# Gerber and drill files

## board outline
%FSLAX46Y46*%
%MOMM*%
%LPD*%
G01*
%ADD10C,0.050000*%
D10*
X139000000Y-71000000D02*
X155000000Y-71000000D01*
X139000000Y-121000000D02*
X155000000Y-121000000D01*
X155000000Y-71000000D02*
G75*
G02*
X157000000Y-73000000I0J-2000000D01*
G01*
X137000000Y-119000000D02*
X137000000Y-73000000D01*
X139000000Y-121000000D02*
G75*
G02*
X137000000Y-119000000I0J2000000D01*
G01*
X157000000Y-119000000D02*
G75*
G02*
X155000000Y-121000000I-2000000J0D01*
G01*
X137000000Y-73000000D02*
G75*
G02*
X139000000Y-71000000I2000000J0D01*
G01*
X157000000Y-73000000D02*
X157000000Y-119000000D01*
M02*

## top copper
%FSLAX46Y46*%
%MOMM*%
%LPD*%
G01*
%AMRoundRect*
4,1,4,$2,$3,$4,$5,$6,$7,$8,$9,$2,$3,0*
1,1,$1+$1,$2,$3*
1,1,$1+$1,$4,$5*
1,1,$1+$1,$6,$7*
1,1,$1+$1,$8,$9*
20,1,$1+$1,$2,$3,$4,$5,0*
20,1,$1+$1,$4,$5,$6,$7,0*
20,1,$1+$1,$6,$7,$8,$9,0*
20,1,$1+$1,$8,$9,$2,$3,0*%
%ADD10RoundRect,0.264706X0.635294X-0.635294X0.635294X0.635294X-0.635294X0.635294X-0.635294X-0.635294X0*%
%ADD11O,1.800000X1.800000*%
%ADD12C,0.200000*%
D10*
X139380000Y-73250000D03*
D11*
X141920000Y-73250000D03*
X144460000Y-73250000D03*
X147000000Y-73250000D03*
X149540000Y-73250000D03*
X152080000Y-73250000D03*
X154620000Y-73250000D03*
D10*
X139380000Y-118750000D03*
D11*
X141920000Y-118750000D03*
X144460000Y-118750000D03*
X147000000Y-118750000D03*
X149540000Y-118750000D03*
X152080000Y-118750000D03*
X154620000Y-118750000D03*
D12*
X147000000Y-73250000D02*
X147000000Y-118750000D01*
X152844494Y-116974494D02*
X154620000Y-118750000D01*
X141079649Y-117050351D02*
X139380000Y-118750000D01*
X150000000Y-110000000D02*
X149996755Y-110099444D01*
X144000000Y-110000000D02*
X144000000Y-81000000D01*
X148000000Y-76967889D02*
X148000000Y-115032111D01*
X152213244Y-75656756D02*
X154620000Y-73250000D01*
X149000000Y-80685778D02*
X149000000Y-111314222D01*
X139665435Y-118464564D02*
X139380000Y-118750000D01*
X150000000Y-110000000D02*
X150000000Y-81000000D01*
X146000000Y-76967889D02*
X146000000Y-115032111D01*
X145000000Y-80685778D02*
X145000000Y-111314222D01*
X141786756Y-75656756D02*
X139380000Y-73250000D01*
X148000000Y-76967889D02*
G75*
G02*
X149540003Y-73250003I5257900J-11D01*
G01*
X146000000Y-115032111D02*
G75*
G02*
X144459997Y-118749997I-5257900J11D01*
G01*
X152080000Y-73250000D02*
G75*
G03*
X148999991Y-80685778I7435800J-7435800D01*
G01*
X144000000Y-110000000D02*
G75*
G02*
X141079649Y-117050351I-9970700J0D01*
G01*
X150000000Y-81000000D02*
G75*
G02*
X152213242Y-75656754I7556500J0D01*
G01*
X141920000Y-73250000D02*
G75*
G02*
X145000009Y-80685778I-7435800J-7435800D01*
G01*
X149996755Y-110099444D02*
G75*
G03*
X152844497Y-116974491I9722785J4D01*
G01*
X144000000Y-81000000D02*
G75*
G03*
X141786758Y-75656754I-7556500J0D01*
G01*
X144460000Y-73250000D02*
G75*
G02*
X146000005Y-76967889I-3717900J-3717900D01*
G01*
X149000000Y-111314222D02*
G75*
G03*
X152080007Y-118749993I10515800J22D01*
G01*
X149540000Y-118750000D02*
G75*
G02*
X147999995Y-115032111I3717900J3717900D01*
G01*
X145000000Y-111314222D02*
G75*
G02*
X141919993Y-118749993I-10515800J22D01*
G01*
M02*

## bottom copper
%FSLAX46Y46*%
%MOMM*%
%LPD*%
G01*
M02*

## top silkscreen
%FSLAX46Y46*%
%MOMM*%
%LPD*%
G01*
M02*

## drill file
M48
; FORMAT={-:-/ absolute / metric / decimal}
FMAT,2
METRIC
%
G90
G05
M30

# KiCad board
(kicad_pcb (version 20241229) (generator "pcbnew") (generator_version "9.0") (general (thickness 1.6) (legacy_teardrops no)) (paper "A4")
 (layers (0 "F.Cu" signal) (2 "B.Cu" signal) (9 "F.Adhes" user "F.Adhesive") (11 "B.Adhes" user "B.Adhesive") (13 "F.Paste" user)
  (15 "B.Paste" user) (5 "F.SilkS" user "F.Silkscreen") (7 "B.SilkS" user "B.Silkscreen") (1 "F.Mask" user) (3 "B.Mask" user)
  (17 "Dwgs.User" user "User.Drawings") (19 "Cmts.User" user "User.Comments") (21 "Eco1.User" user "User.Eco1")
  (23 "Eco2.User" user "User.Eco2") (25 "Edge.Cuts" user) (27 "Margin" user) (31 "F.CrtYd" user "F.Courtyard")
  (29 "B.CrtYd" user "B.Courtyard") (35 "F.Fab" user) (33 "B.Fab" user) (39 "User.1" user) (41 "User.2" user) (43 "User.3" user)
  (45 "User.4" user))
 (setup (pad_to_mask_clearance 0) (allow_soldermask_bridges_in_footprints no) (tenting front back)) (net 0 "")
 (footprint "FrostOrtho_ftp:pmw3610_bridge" (layer "F.Cu") (at 147 73.25 90)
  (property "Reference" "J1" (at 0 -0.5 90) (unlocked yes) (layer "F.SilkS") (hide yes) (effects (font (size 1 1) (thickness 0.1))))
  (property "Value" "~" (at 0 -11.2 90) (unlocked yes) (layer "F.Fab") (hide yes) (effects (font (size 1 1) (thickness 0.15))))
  (pad "1" smd roundrect (at 0 -7.62 90) (size 1.8 1.8) (layers "F.Cu" "F.Mask") (roundrect_rratio 0.1470588235))
  (pad "2" smd oval (at 0 -5.08 90) (size 1.8 1.8) (layers "F.Cu" "F.Mask"))
  (pad "3" smd oval (at 0 -2.54 90) (size 1.8 1.8) (layers "F.Cu" "F.Mask"))
  (pad "4" smd oval (at 0 0 90) (size 1.8 1.8) (layers "F.Cu" "F.Mask"))
  (pad "5" smd oval (at 0 2.54 90) (size 1.8 1.8) (layers "F.Cu" "F.Mask"))
  (pad "6" smd oval (at 0 5.08 90) (size 1.8 1.8) (layers "F.Cu" "F.Mask"))
  (pad "7" smd oval (at 0 7.62 90) (size 1.8 1.8) (layers "F.Cu" "F.Mask")))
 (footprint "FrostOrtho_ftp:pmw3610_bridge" (layer "F.Cu") (at 147 118.75 90)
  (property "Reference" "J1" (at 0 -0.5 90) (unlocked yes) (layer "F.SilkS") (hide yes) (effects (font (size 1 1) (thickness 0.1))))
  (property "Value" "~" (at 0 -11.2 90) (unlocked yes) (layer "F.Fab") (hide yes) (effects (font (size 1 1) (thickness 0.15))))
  (pad "1" smd roundrect (at 0 -7.62 90) (size 1.8 1.8) (layers "F.Cu" "F.Mask") (roundrect_rratio 0.1470588235))
  (pad "2" smd oval (at 0 -5.08 90) (size 1.8 1.8) (layers "F.Cu" "F.Mask"))
  (pad "3" smd oval (at 0 -2.54 90) (size 1.8 1.8) (layers "F.Cu" "F.Mask"))
  (pad "4" smd oval (at 0 0 90) (size 1.8 1.8) (layers "F.Cu" "F.Mask"))
  (pad "5" smd oval (at 0 2.54 90) (size 1.8 1.8) (layers "F.Cu" "F.Mask"))
  (pad "6" smd oval (at 0 5.08 90) (size 1.8 1.8) (layers "F.Cu" "F.Mask"))
  (pad "7" smd oval (at 0 7.62 90) (size 1.8 1.8) (layers "F.Cu" "F.Mask")))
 (gr_line (start 139 71) (end 155 71) (stroke (width 0.05) (type default)) (layer "Edge.Cuts"))
 (gr_line (start 139 121) (end 155 121) (stroke (width 0.05) (type default)) (layer "Edge.Cuts"))
 (gr_arc (start 155 71) (mid 156.414214 71.585786) (end 157 73) (stroke (width 0.05) (type default)) (layer "Edge.Cuts"))
 (gr_line (start 137 119) (end 137 73) (stroke (width 0.05) (type default)) (layer "Edge.Cuts"))
 (gr_arc (start 139 121) (mid 137.585786 120.414214) (end 137 119) (stroke (width 0.05) (type default)) (layer "Edge.Cuts"))
 (gr_arc (start 157 119) (mid 156.414214 120.414214) (end 155 121) (stroke (width 0.05) (type default)) (layer "Edge.Cuts"))
 (gr_arc (start 137 73) (mid 137.585786 71.585786) (end 139 71) (stroke (width 0.05) (type default)) (layer "Edge.Cuts"))
 (gr_line (start 157 73) (end 157 119) (stroke (width 0.05) (type default)) (layer "Edge.Cuts"))
 (segment (start 147 73.25) (end 147 118.75) (width 0.2) (layer "F.Cu") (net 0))
 (segment (start 152.844494 116.974494) (end 154.62 118.75) (width 0.2) (layer "F.Cu") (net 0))
 (segment (start 141.079649 117.050351) (end 139.38 118.75) (width 0.2) (layer "F.Cu") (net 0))
 (segment (start 150 110) (end 149.996755 110.099444) (width 0.2) (layer "F.Cu") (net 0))
 (segment (start 144 110) (end 144 81) (width 0.2) (layer "F.Cu") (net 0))
 (segment (start 148 76.967889) (end 148 115.032111) (width 0.2) (layer "F.Cu") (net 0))
 (segment (start 152.213244 75.656756) (end 154.62 73.25) (width 0.2) (layer "F.Cu") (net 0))
 (segment (start 149 80.685778) (end 149 111.314222) (width 0.2) (layer "F.Cu") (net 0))
 (segment (start 139.665435 118.464564) (end 139.38 118.75) (width 0.2) (layer "F.Cu") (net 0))
 (segment (start 150 110) (end 150 81) (width 0.2) (layer "F.Cu") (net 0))
 (segment (start 146 76.967889) (end 146 115.032111) (width 0.2) (layer "F.Cu") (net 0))
 (segment (start 145 80.685778) (end 145 111.314222) (width 0.2) (layer "F.Cu") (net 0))
 (segment (start 141.786756 75.656756) (end 139.38 73.25) (width 0.2) (layer "F.Cu") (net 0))
 (arc (start 148 76.967889) (mid 148.400233 74.955782) (end 149.54 73.25) (width 0.2) (layer "F.Cu") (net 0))
 (arc (start 146 115.032111) (mid 145.599767 117.044218) (end 144.46 118.75) (width 0.2) (layer "F.Cu") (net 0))
 (arc (start 152.08 73.25) (mid 149.800466 76.661564) (end 149 80.685778) (width 0.2) (layer "F.Cu") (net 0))
 (arc (start 144 110) (mid 143.241026 113.815622) (end 141.079649 117.050351) (width 0.2) (layer "F.Cu") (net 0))
 (arc (start 150 81) (mid 150.575203 78.108257) (end 152.213244 75.656756) (width 0.2) (layer "F.Cu") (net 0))
 (arc (start 141.92 73.25) (mid 144.199534 76.661564) (end 145 80.685778) (width 0.2) (layer "F.Cu") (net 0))
 (arc (start 149.996755 110.099444) (mid 150.736858 113.820194) (end 152.844494 116.974494) (width 0.2) (layer "F.Cu") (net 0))
 (arc (start 144 81) (mid 143.424797 78.108257) (end 141.786756 75.656756) (width 0.2) (layer "F.Cu") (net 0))
 (arc (start 144.46 73.25) (mid 145.599767 74.955782) (end 146 76.967889) (width 0.2) (layer "F.Cu") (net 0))
 (arc (start 149 111.314222) (mid 149.800466 115.338436) (end 152.08 118.75) (width 0.2) (layer "F.Cu") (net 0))
 (arc (start 149.54 118.75) (mid 148.400233 117.044218) (end 148 115.032111) (width 0.2) (layer "F.Cu") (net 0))
 (arc (start 145 111.314222) (mid 144.199534 115.338436) (end 141.92 118.75) (width 0.2) (layer "F.Cu") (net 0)))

